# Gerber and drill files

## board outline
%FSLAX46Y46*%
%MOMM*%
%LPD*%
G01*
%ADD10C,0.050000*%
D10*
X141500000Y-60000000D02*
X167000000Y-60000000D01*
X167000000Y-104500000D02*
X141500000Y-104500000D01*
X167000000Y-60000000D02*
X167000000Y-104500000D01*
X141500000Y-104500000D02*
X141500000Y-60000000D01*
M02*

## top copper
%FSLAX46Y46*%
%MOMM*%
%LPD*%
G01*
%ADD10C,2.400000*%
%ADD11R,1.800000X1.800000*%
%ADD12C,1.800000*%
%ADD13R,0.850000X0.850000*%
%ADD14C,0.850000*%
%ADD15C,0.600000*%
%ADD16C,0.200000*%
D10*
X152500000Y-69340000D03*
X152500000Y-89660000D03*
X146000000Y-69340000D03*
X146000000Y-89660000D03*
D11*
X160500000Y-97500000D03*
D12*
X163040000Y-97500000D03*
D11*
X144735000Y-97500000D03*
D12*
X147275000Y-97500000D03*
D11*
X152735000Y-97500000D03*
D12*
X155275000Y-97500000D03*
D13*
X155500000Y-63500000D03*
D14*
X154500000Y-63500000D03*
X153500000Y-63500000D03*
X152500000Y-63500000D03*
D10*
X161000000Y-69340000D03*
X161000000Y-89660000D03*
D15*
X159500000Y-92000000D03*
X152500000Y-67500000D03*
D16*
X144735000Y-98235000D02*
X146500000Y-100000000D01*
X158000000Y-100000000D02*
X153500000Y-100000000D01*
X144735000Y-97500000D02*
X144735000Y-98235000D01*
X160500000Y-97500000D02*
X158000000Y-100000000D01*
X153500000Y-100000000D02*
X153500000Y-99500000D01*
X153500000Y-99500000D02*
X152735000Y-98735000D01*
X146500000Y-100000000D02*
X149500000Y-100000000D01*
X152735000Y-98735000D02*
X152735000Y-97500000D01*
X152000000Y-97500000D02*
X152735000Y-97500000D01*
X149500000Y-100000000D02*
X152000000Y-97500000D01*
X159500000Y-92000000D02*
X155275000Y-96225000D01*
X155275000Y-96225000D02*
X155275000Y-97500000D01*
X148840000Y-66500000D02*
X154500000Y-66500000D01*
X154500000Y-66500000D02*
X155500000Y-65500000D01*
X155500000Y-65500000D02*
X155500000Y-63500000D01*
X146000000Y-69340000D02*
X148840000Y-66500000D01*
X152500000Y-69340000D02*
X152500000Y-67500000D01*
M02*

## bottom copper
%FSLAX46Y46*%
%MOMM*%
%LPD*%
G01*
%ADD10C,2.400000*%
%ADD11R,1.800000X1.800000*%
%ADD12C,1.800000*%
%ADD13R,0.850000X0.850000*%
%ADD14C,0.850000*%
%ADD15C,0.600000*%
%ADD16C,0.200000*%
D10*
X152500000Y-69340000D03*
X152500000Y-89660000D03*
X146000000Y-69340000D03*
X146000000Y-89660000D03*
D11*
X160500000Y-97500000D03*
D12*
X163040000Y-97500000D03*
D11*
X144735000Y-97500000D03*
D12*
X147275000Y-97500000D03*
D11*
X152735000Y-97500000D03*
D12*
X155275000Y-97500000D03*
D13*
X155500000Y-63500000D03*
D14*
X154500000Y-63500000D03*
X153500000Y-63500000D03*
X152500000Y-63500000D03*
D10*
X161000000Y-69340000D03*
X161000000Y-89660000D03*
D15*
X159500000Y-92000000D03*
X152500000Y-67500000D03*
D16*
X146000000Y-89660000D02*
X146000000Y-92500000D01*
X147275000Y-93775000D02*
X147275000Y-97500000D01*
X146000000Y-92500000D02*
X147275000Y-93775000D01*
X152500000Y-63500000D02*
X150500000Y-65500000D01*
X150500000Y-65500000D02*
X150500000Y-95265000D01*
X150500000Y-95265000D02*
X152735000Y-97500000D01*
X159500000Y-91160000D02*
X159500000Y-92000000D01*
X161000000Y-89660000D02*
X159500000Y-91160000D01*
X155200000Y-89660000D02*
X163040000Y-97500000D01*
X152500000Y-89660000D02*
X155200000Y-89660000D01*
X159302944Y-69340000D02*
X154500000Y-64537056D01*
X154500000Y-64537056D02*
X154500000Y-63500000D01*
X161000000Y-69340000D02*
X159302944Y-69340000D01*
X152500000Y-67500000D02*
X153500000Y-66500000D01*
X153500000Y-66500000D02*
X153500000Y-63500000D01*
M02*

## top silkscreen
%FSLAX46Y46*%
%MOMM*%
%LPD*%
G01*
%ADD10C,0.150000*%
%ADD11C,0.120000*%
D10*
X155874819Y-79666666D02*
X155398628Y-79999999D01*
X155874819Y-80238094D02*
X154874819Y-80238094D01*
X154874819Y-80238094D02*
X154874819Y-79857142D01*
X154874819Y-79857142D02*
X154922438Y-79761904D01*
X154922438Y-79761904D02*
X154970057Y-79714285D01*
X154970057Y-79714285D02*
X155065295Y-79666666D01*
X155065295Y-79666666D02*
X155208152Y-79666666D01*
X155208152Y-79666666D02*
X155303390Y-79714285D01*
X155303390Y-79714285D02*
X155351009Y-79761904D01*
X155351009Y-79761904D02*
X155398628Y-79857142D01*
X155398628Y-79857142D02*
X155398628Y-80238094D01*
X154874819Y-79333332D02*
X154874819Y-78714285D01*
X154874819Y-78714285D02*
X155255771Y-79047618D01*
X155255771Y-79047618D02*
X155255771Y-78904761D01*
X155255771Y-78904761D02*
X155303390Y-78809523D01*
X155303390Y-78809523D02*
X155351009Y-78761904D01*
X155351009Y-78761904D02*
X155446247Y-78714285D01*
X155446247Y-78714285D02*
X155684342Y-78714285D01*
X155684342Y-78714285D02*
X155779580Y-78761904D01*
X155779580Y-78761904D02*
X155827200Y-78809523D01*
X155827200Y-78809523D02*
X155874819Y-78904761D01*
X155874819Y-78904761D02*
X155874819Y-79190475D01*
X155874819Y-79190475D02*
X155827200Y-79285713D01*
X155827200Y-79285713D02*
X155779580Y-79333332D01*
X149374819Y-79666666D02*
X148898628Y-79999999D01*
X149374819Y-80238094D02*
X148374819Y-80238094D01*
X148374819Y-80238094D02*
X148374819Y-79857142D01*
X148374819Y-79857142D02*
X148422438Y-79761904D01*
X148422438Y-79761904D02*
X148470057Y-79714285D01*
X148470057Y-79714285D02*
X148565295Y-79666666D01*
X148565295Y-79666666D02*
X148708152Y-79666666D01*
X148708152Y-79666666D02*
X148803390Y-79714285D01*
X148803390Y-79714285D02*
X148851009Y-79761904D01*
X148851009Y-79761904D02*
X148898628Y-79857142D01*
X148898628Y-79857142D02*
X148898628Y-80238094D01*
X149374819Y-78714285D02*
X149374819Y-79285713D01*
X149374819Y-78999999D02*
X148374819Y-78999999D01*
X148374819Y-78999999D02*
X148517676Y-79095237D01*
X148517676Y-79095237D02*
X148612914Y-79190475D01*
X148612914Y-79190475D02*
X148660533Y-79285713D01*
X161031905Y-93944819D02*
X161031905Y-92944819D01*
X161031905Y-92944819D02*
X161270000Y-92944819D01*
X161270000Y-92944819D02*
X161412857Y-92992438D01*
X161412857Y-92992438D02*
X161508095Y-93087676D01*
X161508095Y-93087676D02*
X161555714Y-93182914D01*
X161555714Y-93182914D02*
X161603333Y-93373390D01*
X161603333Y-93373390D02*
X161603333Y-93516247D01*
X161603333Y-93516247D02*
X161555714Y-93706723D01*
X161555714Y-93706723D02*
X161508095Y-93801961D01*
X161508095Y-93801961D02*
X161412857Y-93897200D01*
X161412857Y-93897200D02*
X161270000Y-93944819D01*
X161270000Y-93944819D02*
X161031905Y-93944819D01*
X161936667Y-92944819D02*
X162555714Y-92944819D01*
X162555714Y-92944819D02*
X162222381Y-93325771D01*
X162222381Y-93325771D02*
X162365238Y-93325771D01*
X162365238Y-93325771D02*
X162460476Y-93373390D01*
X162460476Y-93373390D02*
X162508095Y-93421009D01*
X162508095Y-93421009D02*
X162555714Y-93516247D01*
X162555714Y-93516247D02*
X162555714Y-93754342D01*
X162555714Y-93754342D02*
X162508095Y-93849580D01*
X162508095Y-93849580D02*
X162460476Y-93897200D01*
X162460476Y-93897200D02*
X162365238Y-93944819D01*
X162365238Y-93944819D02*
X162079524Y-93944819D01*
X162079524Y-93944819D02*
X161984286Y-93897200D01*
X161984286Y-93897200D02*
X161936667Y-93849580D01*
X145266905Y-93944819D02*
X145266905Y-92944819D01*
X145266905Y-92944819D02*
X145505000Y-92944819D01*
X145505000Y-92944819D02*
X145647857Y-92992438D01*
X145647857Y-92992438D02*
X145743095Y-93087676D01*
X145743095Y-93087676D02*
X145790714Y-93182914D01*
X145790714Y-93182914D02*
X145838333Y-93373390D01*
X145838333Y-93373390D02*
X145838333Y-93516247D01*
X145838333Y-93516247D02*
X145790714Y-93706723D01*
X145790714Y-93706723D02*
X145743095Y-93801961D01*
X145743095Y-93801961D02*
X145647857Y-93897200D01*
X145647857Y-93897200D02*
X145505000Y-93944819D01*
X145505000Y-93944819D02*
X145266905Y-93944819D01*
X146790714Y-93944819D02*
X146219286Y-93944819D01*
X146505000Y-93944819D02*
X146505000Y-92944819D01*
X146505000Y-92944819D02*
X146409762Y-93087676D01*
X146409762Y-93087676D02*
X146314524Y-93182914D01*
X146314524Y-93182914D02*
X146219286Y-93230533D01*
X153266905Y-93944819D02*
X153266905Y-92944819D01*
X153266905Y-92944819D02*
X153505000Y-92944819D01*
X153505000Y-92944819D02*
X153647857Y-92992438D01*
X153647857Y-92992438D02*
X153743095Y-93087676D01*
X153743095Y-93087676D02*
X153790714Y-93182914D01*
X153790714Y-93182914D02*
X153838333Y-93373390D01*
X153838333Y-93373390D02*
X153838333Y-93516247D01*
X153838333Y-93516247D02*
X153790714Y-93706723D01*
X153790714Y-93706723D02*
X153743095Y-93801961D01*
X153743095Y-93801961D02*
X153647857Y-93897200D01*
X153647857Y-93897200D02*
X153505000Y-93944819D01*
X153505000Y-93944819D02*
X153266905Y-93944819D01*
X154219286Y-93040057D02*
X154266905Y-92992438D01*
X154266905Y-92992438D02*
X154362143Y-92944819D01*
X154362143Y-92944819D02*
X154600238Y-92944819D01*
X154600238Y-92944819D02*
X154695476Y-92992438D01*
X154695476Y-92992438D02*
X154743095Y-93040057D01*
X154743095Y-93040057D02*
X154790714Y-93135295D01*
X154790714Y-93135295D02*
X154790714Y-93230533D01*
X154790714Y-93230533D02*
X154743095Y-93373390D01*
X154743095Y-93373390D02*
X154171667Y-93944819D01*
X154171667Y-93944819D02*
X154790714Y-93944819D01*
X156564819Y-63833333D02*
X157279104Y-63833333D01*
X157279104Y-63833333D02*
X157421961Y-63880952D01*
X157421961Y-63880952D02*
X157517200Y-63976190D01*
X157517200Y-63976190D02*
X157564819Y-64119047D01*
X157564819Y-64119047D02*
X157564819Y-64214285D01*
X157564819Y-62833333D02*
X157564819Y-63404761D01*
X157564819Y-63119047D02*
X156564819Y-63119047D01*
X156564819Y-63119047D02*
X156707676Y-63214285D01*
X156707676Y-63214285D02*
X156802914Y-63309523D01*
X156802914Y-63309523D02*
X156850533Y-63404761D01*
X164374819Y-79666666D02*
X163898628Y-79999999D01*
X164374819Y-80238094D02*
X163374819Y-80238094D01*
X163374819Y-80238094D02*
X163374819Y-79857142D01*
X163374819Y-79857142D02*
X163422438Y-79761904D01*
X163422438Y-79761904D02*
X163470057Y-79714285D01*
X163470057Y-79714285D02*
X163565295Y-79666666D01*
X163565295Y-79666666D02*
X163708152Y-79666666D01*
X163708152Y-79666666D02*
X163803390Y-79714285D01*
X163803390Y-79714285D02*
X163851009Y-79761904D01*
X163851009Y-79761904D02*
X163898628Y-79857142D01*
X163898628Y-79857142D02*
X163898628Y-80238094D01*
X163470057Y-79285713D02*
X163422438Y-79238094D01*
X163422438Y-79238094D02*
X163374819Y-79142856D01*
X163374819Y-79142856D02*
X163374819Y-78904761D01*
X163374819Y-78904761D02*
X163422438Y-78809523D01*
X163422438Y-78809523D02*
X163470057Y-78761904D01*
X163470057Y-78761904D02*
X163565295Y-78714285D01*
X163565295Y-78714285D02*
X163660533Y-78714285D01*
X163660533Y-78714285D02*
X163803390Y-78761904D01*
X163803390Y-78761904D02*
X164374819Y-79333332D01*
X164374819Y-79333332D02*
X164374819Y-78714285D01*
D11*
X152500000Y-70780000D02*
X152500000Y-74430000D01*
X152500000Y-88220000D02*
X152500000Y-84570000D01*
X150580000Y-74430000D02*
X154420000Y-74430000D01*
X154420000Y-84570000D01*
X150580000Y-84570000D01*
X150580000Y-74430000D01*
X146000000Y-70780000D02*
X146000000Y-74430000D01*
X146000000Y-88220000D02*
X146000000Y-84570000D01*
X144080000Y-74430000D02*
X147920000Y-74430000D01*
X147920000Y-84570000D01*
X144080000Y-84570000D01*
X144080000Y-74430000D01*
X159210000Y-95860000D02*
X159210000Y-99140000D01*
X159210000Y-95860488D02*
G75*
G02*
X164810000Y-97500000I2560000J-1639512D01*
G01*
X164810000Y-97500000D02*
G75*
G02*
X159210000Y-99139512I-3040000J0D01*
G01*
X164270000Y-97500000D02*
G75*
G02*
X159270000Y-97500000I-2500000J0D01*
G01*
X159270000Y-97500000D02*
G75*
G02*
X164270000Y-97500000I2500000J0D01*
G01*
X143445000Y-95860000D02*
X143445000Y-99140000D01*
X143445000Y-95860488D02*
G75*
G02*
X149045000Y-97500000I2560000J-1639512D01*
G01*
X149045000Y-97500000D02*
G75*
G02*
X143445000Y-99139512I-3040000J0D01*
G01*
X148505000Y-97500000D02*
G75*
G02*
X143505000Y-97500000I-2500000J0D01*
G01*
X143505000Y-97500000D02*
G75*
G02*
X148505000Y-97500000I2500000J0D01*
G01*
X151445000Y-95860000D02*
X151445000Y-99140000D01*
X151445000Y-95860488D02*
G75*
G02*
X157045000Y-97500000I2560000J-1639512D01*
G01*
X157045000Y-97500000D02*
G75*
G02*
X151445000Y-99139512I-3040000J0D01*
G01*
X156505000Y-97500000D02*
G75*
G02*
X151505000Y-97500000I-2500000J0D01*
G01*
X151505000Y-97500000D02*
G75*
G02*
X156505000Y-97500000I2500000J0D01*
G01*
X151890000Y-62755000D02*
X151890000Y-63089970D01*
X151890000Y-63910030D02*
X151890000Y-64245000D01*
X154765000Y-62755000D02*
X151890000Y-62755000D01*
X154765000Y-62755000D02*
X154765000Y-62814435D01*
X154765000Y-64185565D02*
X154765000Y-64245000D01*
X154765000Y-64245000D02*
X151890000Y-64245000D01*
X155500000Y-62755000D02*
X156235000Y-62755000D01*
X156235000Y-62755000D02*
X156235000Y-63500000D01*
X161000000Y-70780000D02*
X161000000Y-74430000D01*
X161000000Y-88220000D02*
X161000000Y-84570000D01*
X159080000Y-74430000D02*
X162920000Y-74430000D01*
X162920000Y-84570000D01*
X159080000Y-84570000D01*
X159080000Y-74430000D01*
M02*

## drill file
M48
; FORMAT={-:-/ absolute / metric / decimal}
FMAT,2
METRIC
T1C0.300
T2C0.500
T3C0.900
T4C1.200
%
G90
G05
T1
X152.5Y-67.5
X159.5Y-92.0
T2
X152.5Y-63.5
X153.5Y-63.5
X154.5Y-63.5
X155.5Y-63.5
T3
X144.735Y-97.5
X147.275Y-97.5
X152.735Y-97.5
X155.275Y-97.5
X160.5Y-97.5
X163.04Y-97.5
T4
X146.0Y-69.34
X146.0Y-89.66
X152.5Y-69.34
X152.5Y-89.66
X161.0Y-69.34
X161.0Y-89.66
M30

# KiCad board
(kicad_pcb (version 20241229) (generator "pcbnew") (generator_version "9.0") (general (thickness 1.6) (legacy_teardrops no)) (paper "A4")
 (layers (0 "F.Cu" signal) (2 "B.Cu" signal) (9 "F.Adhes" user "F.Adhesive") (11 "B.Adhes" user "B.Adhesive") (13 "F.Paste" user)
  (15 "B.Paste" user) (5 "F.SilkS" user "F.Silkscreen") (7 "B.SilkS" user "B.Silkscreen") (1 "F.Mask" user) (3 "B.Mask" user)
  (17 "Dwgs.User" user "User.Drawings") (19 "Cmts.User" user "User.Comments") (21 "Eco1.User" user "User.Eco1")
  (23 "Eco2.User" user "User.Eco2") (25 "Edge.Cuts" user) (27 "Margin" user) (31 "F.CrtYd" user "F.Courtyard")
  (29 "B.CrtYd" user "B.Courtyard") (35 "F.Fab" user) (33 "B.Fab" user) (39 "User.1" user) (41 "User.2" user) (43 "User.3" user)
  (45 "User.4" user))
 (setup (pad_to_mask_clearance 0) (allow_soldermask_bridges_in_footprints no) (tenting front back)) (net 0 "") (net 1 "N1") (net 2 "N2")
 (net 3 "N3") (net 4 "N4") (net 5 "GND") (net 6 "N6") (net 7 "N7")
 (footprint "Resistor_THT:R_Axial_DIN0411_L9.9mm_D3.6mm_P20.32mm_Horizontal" (layer "F.Cu") (at 152.5 69.34 -90)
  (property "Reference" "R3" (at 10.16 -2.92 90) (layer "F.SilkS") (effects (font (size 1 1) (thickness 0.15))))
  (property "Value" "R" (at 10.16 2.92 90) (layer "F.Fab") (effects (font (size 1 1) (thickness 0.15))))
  (fp_line (start 1.44 0) (end 5.09 0) (stroke (width 0.12) (type solid)) (layer "F.SilkS"))
  (fp_line (start 18.88 0) (end 15.23 0) (stroke (width 0.12) (type solid)) (layer "F.SilkS"))
  (fp_rect (start 5.09 -1.92) (end 15.23 1.92) (stroke (width 0.12) (type solid)) (fill no) (layer "F.SilkS"))
  (pad "1" thru_hole circle (at 0 0 270) (size 2.4 2.4) (drill 1.2) (layers "*.Cu" "*.Mask") (remove_unused_layers no) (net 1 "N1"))
  (pad "2" thru_hole circle (at 20.32 0 270) (size 2.4 2.4) (drill 1.2) (layers "*.Cu" "*.Mask") (remove_unused_layers no) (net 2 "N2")))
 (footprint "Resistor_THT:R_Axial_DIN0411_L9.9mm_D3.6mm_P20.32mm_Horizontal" (layer "F.Cu") (at 146 69.34 -90)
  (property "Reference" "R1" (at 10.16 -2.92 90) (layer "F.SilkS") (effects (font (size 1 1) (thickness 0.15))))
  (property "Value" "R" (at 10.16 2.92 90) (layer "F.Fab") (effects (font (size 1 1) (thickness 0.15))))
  (fp_line (start 1.44 0) (end 5.09 0) (stroke (width 0.12) (type solid)) (layer "F.SilkS"))
  (fp_line (start 18.88 0) (end 15.23 0) (stroke (width 0.12) (type solid)) (layer "F.SilkS"))
  (fp_rect (start 5.09 -1.92) (end 15.23 1.92) (stroke (width 0.12) (type solid)) (fill no) (layer "F.SilkS"))
  (pad "1" thru_hole circle (at 0 0 270) (size 2.4 2.4) (drill 1.2) (layers "*.Cu" "*.Mask") (remove_unused_layers no) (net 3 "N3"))
  (pad "2" thru_hole circle (at 20.32 0 270) (size 2.4 2.4) (drill 1.2) (layers "*.Cu" "*.Mask") (remove_unused_layers no) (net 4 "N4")))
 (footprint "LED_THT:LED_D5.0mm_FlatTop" (layer "F.Cu") (at 160.5 97.5)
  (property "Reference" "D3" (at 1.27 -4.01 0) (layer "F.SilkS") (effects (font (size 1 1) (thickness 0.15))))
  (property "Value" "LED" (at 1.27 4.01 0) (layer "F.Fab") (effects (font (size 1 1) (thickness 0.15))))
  (fp_line (start -1.29 -1.64) (end -1.29 1.64) (stroke (width 0.12) (type solid)) (layer "F.SilkS"))
  (fp_arc (start -1.29 -1.639512) (mid 2.124166 -2.917533) (end 4.31 0) (stroke (width 0.12) (type solid)) (layer "F.SilkS"))
  (fp_arc (start 4.31 0) (mid 2.124166 2.917533) (end -1.29 1.639512) (stroke (width 0.12) (type solid)) (layer "F.SilkS"))
  (fp_circle (center 1.27 0) (end 3.77 0) (stroke (width 0.12) (type solid)) (fill no) (layer "F.SilkS"))
  (pad "1" thru_hole rect (at 0 0) (size 1.8 1.8) (drill 0.9) (layers "*.Cu" "*.Mask") (remove_unused_layers no) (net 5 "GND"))
  (pad "2" thru_hole circle (at 2.54 0) (size 1.8 1.8) (drill 0.9) (layers "*.Cu" "*.Mask") (remove_unused_layers no) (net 2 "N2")))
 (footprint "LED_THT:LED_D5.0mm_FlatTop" (layer "F.Cu") (at 144.735 97.5)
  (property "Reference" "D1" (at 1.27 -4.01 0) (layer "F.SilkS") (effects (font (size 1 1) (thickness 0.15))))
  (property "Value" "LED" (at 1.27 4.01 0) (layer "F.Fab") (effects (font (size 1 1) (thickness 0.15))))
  (fp_line (start -1.29 -1.64) (end -1.29 1.64) (stroke (width 0.12) (type solid)) (layer "F.SilkS"))
  (fp_arc (start -1.29 -1.639512) (mid 2.124166 -2.917533) (end 4.31 0) (stroke (width 0.12) (type solid)) (layer "F.SilkS"))
  (fp_arc (start 4.31 0) (mid 2.124166 2.917533) (end -1.29 1.639512) (stroke (width 0.12) (type solid)) (layer "F.SilkS"))
  (fp_circle (center 1.27 0) (end 3.77 0) (stroke (width 0.12) (type solid)) (fill no) (layer "F.SilkS"))
  (pad "1" thru_hole rect (at 0 0) (size 1.8 1.8) (drill 0.9) (layers "*.Cu" "*.Mask") (remove_unused_layers no) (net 5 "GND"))
  (pad "2" thru_hole circle (at 2.54 0) (size 1.8 1.8) (drill 0.9) (layers "*.Cu" "*.Mask") (remove_unused_layers no) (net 4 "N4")))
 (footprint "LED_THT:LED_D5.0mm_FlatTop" (layer "F.Cu") (at 152.735 97.5)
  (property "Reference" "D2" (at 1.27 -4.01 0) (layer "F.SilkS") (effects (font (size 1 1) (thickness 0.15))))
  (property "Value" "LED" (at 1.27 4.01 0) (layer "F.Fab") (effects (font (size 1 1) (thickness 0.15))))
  (fp_line (start -1.29 -1.64) (end -1.29 1.64) (stroke (width 0.12) (type solid)) (layer "F.SilkS"))
  (fp_arc (start -1.29 -1.639512) (mid 2.124166 -2.917533) (end 4.31 0) (stroke (width 0.12) (type solid)) (layer "F.SilkS"))
  (fp_arc (start 4.31 0) (mid 2.124166 2.917533) (end -1.29 1.639512) (stroke (width 0.12) (type solid)) (layer "F.SilkS"))
  (fp_circle (center 1.27 0) (end 3.77 0) (stroke (width 0.12) (type solid)) (fill no) (layer "F.SilkS"))
  (pad "1" thru_hole rect (at 0 0) (size 1.8 1.8) (drill 0.9) (layers "*.Cu" "*.Mask") (remove_unused_layers no) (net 5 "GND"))
  (pad "2" thru_hole circle (at 2.54 0) (size 1.8 1.8) (drill 0.9) (layers "*.Cu" "*.Mask") (remove_unused_layers no) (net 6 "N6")))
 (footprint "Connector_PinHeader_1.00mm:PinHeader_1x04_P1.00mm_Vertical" (layer "F.Cu") (at 155.5 63.5 -90)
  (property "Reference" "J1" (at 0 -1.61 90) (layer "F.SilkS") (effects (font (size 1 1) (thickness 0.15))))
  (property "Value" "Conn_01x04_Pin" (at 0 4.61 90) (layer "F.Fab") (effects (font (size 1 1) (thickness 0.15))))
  (fp_line (start -0.745 3.61) (end -0.41003 3.61) (stroke (width 0.12) (type solid)) (layer "F.SilkS"))
  (fp_line (start 0.41003 3.61) (end 0.745 3.61) (stroke (width 0.12) (type solid)) (layer "F.SilkS"))
  (fp_line (start -0.745 0.735) (end -0.745 3.61) (stroke (width 0.12) (type solid)) (layer "F.SilkS"))
  (fp_line (start -0.745 0.735) (end -0.685565 0.735) (stroke (width 0.12) (type solid)) (layer "F.SilkS"))
  (fp_line (start 0.685565 0.735) (end 0.745 0.735) (stroke (width 0.12) (type solid)) (layer "F.SilkS"))
  (fp_line (start 0.745 0.735) (end 0.745 3.61) (stroke (width 0.12) (type solid)) (layer "F.SilkS"))
  (fp_line (start -0.745 0) (end -0.745 -0.735) (stroke (width 0.12) (type solid)) (layer "F.SilkS"))
  (fp_line (start -0.745 -0.735) (end 0 -0.735) (stroke (width 0.12) (type solid)) (layer "F.SilkS"))
  (pad "1" thru_hole rect (at 0 0 270) (size 0.85 0.85) (drill 0.5) (layers "*.Cu" "*.Mask") (remove_unused_layers no) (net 3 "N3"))
  (pad "2" thru_hole circle (at 0 1 270) (size 0.85 0.85) (drill 0.5) (layers "*.Cu" "*.Mask") (remove_unused_layers no) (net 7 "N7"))
  (pad "3" thru_hole circle (at 0 2 270) (size 0.85 0.85) (drill 0.5) (layers "*.Cu" "*.Mask") (remove_unused_layers no) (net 1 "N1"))
  (pad "4" thru_hole circle (at 0 3 270) (size 0.85 0.85) (drill 0.5) (layers "*.Cu" "*.Mask") (remove_unused_layers no) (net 5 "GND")))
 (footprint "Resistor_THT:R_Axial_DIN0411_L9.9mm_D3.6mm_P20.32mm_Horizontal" (layer "F.Cu") (at 161 69.34 -90)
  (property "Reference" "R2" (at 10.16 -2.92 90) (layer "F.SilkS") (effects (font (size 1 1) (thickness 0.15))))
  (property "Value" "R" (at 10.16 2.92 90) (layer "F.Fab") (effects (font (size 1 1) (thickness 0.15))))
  (fp_line (start 1.44 0) (end 5.09 0) (stroke (width 0.12) (type solid)) (layer "F.SilkS"))
  (fp_line (start 18.88 0) (end 15.23 0) (stroke (width 0.12) (type solid)) (layer "F.SilkS"))
  (fp_rect (start 5.09 -1.92) (end 15.23 1.92) (stroke (width 0.12) (type solid)) (fill no) (layer "F.SilkS"))
  (pad "1" thru_hole circle (at 0 0 270) (size 2.4 2.4) (drill 1.2) (layers "*.Cu" "*.Mask") (remove_unused_layers no) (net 7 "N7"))
  (pad "2" thru_hole circle (at 20.32 0 270) (size 2.4 2.4) (drill 1.2) (layers "*.Cu" "*.Mask") (remove_unused_layers no) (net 6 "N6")))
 (gr_line (start 141.5 60) (end 167 60) (stroke (width 0.05) (type default)) (layer "Edge.Cuts"))
 (gr_line (start 167 104.5) (end 141.5 104.5) (stroke (width 0.05) (type default)) (layer "Edge.Cuts"))
 (gr_line (start 167 60) (end 167 104.5) (stroke (width 0.05) (type default)) (layer "Edge.Cuts"))
 (gr_line (start 141.5 104.5) (end 141.5 60) (stroke (width 0.05) (type default)) (layer "Edge.Cuts"))
 (segment (start 146 89.66) (end 146 92.5) (width 0.2) (layer "B.Cu") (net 4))
 (segment (start 147.275 93.775) (end 147.275 97.5) (width 0.2) (layer "B.Cu") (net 4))
 (segment (start 146 92.5) (end 147.275 93.775) (width 0.2) (layer "B.Cu") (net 4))
 (segment (start 144.735 98.235) (end 146.5 100) (width 0.2) (layer "F.Cu") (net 5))
 (segment (start 158 100) (end 153.5 100) (width 0.2) (layer "F.Cu") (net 5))
 (segment (start 144.735 97.5) (end 144.735 98.235) (width 0.2) (layer "F.Cu") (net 5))
 (segment (start 160.5 97.5) (end 158 100) (width 0.2) (layer "F.Cu") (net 5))
 (segment (start 153.5 100) (end 153.5 99.5) (width 0.2) (layer "F.Cu") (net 5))
 (segment (start 153.5 99.5) (end 152.735 98.735) (width 0.2) (layer "F.Cu") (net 5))
 (segment (start 146.5 100) (end 149.5 100) (width 0.2) (layer "F.Cu") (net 5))
 (segment (start 152.735 98.735) (end 152.735 97.5) (width 0.2) (layer "F.Cu") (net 5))
 (segment (start 152 97.5) (end 152.735 97.5) (width 0.2) (layer "F.Cu") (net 5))
 (segment (start 149.5 100) (end 152 97.5) (width 0.2) (layer "F.Cu") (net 5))
 (segment (start 152.5 63.5) (end 150.5 65.5) (width 0.2) (layer "B.Cu") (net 5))
 (segment (start 150.5 65.5) (end 150.5 95.265) (width 0.2) (layer "B.Cu") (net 5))
 (segment (start 150.5 95.265) (end 152.735 97.5) (width 0.2) (layer "B.Cu") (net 5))
 (segment (start 159.5 92) (end 155.275 96.225) (width 0.2) (layer "F.Cu") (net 6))
 (segment (start 155.275 96.225) (end 155.275 97.5) (width 0.2) (layer "F.Cu") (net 6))
 (via (at 159.5 92) (size 0.6) (drill 0.3) (layers "F.Cu" "B.Cu") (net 6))
 (segment (start 159.5 91.16) (end 159.5 92) (width 0.2) (layer "B.Cu") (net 6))
 (segment (start 161 89.66) (end 159.5 91.16) (width 0.2) (layer "B.Cu") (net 6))
 (segment (start 155.2 89.66) (end 163.04 97.5) (width 0.2) (layer "B.Cu") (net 2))
 (segment (start 152.5 89.66) (end 155.2 89.66) (width 0.2) (layer "B.Cu") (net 2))
 (segment (start 159.302944 69.34) (end 154.5 64.537056) (width 0.2) (layer "B.Cu") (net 7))
 (segment (start 154.5 64.537056) (end 154.5 63.5) (width 0.2) (layer "B.Cu") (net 7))
 (segment (start 161 69.34) (end 159.302944 69.34) (width 0.2) (layer "B.Cu") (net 7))
 (segment (start 148.84 66.5) (end 154.5 66.5) (width 0.2) (layer "F.Cu") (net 3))
 (segment (start 154.5 66.5) (end 155.5 65.5) (width 0.2) (layer "F.Cu") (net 3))
 (segment (start 155.5 65.5) (end 155.5 63.5) (width 0.2) (layer "F.Cu") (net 3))
 (segment (start 146 69.34) (end 148.84 66.5) (width 0.2) (layer "F.Cu") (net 3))
 (segment (start 152.5 69.34) (end 152.5 67.5) (width 0.2) (layer "F.Cu") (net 1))
 (via (at 152.5 67.5) (size 0.6) (drill 0.3) (layers "F.Cu" "B.Cu") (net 1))
 (segment (start 152.5 67.5) (end 153.5 66.5) (width 0.2) (layer "B.Cu") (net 1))
 (segment (start 153.5 66.5) (end 153.5 63.5) (width 0.2) (layer "B.Cu") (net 1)))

